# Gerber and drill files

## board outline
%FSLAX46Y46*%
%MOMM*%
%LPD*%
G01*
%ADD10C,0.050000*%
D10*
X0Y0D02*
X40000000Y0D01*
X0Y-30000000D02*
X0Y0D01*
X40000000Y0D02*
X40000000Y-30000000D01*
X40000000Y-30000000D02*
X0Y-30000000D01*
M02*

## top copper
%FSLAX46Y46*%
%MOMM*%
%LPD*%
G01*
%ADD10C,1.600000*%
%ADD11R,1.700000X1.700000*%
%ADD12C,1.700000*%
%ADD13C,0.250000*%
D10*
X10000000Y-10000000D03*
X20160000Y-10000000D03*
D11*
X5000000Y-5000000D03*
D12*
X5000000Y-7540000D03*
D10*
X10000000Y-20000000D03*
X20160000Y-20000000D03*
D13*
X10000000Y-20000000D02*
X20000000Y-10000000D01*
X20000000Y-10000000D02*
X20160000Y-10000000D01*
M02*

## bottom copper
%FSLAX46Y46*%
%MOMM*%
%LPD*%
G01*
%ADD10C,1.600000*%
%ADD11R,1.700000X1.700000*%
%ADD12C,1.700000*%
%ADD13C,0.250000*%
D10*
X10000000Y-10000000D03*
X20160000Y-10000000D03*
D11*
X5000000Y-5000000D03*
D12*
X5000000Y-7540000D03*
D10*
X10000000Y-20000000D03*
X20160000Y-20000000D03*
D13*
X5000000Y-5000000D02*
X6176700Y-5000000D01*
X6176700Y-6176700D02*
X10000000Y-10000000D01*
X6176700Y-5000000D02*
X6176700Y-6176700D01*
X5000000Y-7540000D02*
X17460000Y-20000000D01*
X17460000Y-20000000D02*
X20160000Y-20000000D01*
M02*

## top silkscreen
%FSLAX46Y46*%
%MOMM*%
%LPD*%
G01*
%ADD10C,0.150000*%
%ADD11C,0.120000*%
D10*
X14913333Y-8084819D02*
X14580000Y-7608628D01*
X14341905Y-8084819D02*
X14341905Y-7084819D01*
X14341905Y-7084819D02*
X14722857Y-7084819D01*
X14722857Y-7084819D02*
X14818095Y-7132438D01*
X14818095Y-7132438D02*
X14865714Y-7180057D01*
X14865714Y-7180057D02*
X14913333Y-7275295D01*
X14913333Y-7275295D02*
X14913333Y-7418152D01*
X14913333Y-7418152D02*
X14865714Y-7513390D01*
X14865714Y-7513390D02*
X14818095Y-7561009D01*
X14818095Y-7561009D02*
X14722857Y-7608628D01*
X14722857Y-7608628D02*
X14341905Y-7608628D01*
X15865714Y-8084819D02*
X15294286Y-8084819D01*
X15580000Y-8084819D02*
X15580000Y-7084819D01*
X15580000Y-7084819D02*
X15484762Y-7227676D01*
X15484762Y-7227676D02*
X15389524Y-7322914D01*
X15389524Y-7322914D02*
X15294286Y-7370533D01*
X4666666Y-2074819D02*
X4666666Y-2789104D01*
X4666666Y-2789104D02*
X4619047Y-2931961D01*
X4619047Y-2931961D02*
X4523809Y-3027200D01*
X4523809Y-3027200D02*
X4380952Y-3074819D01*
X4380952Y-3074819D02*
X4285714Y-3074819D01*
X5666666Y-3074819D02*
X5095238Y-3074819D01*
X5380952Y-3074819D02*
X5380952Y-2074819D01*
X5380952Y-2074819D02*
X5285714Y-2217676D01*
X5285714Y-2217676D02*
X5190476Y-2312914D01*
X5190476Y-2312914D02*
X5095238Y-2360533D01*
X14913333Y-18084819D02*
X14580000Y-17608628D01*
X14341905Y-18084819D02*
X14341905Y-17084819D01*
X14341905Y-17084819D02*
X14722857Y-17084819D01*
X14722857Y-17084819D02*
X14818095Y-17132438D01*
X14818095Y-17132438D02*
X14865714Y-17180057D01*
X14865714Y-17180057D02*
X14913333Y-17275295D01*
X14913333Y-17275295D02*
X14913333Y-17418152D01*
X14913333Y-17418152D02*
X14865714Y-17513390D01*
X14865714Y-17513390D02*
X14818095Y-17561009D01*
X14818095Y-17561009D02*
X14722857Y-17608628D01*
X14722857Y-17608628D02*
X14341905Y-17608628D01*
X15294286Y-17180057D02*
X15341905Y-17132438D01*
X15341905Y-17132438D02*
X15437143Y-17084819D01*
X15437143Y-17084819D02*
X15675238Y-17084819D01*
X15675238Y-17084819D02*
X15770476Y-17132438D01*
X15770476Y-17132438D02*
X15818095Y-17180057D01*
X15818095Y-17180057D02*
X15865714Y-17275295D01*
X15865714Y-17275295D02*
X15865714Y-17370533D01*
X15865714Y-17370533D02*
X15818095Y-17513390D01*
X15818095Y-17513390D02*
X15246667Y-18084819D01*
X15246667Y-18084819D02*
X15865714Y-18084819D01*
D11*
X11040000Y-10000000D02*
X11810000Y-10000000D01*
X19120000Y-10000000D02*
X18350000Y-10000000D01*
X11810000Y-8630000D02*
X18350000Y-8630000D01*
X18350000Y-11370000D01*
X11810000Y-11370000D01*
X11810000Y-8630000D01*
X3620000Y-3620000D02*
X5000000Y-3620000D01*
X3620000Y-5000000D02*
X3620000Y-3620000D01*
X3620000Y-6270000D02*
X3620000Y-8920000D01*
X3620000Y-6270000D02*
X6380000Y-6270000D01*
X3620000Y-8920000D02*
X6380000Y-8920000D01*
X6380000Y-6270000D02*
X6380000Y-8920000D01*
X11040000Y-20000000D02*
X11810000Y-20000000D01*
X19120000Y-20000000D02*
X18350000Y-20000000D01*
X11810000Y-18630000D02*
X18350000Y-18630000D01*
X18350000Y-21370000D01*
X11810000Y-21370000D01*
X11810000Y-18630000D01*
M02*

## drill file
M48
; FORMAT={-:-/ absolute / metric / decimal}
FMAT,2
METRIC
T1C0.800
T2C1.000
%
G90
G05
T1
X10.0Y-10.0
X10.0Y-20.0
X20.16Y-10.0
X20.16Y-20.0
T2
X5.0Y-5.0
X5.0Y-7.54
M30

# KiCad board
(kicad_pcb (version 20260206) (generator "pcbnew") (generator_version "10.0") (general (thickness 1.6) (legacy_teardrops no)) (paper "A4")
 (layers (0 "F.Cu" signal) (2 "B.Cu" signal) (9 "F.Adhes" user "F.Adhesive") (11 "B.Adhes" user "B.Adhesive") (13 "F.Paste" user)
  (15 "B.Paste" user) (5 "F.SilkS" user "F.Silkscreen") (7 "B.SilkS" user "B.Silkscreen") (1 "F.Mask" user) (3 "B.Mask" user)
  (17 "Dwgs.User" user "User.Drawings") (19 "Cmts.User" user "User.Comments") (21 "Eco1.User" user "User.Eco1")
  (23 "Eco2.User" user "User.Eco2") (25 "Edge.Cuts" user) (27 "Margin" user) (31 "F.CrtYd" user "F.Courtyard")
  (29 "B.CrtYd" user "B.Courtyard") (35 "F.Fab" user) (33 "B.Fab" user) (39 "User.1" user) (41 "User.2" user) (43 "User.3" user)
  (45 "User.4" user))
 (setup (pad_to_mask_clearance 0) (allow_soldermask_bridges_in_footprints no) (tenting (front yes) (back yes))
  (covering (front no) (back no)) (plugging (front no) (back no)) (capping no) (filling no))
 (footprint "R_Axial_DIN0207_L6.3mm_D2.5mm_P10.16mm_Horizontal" (layer "F.Cu") (at 10 10)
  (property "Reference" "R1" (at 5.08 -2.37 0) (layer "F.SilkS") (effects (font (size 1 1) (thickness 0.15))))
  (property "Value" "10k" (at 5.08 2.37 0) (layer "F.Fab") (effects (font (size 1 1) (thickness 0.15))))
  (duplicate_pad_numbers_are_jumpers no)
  (fp_line (start 1.04 0) (end 1.81 0) (stroke (width 0.12) (type solid)) (layer "F.SilkS"))
  (fp_line (start 9.12 0) (end 8.35 0) (stroke (width 0.12) (type solid)) (layer "F.SilkS"))
  (fp_rect (start 1.81 -1.37) (end 8.35 1.37) (stroke (width 0.12) (type solid)) (fill no) (layer "F.SilkS"))
  (pad "1" thru_hole circle (at 0 0) (size 1.6 1.6) (drill 0.8) (layers "*.Cu" "*.Mask") (remove_unused_layers no) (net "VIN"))
  (pad "2" thru_hole circle (at 10.16 0) (size 1.6 1.6) (drill 0.8) (layers "*.Cu" "*.Mask") (remove_unused_layers no) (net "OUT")))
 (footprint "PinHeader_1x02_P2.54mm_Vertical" (layer "F.Cu") (at 5 5)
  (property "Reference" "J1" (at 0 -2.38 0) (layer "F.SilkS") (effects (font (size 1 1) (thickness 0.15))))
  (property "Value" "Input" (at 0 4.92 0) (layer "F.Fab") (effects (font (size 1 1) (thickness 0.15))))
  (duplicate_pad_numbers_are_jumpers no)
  (fp_line (start -1.38 -1.38) (end 0 -1.38) (stroke (width 0.12) (type solid)) (layer "F.SilkS"))
  (fp_line (start -1.38 0) (end -1.38 -1.38) (stroke (width 0.12) (type solid)) (layer "F.SilkS"))
  (fp_line (start -1.38 1.27) (end -1.38 3.92) (stroke (width 0.12) (type solid)) (layer "F.SilkS"))
  (fp_line (start -1.38 1.27) (end 1.38 1.27) (stroke (width 0.12) (type solid)) (layer "F.SilkS"))
  (fp_line (start -1.38 3.92) (end 1.38 3.92) (stroke (width 0.12) (type solid)) (layer "F.SilkS"))
  (fp_line (start 1.38 1.27) (end 1.38 3.92) (stroke (width 0.12) (type solid)) (layer "F.SilkS"))
  (pad "1" thru_hole rect (at 0 0) (size 1.7 1.7) (drill 1) (layers "*.Cu" "*.Mask") (remove_unused_layers no) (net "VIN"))
  (pad "2" thru_hole circle (at 0 2.54) (size 1.7 1.7) (drill 1) (layers "*.Cu" "*.Mask") (remove_unused_layers no) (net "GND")))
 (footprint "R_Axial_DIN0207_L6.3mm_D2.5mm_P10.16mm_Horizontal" (layer "F.Cu") (at 10 20)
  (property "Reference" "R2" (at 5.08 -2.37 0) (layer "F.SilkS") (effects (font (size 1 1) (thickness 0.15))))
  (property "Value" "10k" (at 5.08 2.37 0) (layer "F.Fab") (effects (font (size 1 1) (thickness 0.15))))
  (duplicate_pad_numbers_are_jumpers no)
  (fp_line (start 1.04 0) (end 1.81 0) (stroke (width 0.12) (type solid)) (layer "F.SilkS"))
  (fp_line (start 9.12 0) (end 8.35 0) (stroke (width 0.12) (type solid)) (layer "F.SilkS"))
  (fp_rect (start 1.81 -1.37) (end 8.35 1.37) (stroke (width 0.12) (type solid)) (fill no) (layer "F.SilkS"))
  (pad "1" thru_hole circle (at 0 0) (size 1.6 1.6) (drill 0.8) (layers "*.Cu" "*.Mask") (remove_unused_layers no) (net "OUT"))
  (pad "2" thru_hole circle (at 10.16 0) (size 1.6 1.6) (drill 0.8) (layers "*.Cu" "*.Mask") (remove_unused_layers no) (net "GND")))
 (gr_line (start 0 0) (end 40 0) (stroke (width 0.05) (type default)) (layer "Edge.Cuts"))
 (gr_line (start 0 30) (end 0 0) (stroke (width 0.05) (type default)) (layer "Edge.Cuts"))
 (gr_line (start 40 0) (end 40 30) (stroke (width 0.05) (type default)) (layer "Edge.Cuts"))
 (gr_line (start 40 30) (end 0 30) (stroke (width 0.05) (type default)) (layer "Edge.Cuts"))
 (segment (start 5 5) (end 6.1767 5) (width 0.25) (layer "B.Cu") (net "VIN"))
 (segment (start 6.1767 6.1767) (end 10 10) (width 0.25) (layer "B.Cu") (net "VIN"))
 (segment (start 6.1767 5) (end 6.1767 6.1767) (width 0.25) (layer "B.Cu") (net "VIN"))
 (segment (start 10 20) (end 20 10) (width 0.25) (layer "F.Cu") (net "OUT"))
 (segment (start 20 10) (end 20.16 10) (width 0.25) (layer "F.Cu") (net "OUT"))
 (segment (start 5 7.54) (end 17.46 20) (width 0.25) (layer "B.Cu") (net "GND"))
 (segment (start 17.46 20) (end 20.16 20) (width 0.25) (layer "B.Cu") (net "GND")))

